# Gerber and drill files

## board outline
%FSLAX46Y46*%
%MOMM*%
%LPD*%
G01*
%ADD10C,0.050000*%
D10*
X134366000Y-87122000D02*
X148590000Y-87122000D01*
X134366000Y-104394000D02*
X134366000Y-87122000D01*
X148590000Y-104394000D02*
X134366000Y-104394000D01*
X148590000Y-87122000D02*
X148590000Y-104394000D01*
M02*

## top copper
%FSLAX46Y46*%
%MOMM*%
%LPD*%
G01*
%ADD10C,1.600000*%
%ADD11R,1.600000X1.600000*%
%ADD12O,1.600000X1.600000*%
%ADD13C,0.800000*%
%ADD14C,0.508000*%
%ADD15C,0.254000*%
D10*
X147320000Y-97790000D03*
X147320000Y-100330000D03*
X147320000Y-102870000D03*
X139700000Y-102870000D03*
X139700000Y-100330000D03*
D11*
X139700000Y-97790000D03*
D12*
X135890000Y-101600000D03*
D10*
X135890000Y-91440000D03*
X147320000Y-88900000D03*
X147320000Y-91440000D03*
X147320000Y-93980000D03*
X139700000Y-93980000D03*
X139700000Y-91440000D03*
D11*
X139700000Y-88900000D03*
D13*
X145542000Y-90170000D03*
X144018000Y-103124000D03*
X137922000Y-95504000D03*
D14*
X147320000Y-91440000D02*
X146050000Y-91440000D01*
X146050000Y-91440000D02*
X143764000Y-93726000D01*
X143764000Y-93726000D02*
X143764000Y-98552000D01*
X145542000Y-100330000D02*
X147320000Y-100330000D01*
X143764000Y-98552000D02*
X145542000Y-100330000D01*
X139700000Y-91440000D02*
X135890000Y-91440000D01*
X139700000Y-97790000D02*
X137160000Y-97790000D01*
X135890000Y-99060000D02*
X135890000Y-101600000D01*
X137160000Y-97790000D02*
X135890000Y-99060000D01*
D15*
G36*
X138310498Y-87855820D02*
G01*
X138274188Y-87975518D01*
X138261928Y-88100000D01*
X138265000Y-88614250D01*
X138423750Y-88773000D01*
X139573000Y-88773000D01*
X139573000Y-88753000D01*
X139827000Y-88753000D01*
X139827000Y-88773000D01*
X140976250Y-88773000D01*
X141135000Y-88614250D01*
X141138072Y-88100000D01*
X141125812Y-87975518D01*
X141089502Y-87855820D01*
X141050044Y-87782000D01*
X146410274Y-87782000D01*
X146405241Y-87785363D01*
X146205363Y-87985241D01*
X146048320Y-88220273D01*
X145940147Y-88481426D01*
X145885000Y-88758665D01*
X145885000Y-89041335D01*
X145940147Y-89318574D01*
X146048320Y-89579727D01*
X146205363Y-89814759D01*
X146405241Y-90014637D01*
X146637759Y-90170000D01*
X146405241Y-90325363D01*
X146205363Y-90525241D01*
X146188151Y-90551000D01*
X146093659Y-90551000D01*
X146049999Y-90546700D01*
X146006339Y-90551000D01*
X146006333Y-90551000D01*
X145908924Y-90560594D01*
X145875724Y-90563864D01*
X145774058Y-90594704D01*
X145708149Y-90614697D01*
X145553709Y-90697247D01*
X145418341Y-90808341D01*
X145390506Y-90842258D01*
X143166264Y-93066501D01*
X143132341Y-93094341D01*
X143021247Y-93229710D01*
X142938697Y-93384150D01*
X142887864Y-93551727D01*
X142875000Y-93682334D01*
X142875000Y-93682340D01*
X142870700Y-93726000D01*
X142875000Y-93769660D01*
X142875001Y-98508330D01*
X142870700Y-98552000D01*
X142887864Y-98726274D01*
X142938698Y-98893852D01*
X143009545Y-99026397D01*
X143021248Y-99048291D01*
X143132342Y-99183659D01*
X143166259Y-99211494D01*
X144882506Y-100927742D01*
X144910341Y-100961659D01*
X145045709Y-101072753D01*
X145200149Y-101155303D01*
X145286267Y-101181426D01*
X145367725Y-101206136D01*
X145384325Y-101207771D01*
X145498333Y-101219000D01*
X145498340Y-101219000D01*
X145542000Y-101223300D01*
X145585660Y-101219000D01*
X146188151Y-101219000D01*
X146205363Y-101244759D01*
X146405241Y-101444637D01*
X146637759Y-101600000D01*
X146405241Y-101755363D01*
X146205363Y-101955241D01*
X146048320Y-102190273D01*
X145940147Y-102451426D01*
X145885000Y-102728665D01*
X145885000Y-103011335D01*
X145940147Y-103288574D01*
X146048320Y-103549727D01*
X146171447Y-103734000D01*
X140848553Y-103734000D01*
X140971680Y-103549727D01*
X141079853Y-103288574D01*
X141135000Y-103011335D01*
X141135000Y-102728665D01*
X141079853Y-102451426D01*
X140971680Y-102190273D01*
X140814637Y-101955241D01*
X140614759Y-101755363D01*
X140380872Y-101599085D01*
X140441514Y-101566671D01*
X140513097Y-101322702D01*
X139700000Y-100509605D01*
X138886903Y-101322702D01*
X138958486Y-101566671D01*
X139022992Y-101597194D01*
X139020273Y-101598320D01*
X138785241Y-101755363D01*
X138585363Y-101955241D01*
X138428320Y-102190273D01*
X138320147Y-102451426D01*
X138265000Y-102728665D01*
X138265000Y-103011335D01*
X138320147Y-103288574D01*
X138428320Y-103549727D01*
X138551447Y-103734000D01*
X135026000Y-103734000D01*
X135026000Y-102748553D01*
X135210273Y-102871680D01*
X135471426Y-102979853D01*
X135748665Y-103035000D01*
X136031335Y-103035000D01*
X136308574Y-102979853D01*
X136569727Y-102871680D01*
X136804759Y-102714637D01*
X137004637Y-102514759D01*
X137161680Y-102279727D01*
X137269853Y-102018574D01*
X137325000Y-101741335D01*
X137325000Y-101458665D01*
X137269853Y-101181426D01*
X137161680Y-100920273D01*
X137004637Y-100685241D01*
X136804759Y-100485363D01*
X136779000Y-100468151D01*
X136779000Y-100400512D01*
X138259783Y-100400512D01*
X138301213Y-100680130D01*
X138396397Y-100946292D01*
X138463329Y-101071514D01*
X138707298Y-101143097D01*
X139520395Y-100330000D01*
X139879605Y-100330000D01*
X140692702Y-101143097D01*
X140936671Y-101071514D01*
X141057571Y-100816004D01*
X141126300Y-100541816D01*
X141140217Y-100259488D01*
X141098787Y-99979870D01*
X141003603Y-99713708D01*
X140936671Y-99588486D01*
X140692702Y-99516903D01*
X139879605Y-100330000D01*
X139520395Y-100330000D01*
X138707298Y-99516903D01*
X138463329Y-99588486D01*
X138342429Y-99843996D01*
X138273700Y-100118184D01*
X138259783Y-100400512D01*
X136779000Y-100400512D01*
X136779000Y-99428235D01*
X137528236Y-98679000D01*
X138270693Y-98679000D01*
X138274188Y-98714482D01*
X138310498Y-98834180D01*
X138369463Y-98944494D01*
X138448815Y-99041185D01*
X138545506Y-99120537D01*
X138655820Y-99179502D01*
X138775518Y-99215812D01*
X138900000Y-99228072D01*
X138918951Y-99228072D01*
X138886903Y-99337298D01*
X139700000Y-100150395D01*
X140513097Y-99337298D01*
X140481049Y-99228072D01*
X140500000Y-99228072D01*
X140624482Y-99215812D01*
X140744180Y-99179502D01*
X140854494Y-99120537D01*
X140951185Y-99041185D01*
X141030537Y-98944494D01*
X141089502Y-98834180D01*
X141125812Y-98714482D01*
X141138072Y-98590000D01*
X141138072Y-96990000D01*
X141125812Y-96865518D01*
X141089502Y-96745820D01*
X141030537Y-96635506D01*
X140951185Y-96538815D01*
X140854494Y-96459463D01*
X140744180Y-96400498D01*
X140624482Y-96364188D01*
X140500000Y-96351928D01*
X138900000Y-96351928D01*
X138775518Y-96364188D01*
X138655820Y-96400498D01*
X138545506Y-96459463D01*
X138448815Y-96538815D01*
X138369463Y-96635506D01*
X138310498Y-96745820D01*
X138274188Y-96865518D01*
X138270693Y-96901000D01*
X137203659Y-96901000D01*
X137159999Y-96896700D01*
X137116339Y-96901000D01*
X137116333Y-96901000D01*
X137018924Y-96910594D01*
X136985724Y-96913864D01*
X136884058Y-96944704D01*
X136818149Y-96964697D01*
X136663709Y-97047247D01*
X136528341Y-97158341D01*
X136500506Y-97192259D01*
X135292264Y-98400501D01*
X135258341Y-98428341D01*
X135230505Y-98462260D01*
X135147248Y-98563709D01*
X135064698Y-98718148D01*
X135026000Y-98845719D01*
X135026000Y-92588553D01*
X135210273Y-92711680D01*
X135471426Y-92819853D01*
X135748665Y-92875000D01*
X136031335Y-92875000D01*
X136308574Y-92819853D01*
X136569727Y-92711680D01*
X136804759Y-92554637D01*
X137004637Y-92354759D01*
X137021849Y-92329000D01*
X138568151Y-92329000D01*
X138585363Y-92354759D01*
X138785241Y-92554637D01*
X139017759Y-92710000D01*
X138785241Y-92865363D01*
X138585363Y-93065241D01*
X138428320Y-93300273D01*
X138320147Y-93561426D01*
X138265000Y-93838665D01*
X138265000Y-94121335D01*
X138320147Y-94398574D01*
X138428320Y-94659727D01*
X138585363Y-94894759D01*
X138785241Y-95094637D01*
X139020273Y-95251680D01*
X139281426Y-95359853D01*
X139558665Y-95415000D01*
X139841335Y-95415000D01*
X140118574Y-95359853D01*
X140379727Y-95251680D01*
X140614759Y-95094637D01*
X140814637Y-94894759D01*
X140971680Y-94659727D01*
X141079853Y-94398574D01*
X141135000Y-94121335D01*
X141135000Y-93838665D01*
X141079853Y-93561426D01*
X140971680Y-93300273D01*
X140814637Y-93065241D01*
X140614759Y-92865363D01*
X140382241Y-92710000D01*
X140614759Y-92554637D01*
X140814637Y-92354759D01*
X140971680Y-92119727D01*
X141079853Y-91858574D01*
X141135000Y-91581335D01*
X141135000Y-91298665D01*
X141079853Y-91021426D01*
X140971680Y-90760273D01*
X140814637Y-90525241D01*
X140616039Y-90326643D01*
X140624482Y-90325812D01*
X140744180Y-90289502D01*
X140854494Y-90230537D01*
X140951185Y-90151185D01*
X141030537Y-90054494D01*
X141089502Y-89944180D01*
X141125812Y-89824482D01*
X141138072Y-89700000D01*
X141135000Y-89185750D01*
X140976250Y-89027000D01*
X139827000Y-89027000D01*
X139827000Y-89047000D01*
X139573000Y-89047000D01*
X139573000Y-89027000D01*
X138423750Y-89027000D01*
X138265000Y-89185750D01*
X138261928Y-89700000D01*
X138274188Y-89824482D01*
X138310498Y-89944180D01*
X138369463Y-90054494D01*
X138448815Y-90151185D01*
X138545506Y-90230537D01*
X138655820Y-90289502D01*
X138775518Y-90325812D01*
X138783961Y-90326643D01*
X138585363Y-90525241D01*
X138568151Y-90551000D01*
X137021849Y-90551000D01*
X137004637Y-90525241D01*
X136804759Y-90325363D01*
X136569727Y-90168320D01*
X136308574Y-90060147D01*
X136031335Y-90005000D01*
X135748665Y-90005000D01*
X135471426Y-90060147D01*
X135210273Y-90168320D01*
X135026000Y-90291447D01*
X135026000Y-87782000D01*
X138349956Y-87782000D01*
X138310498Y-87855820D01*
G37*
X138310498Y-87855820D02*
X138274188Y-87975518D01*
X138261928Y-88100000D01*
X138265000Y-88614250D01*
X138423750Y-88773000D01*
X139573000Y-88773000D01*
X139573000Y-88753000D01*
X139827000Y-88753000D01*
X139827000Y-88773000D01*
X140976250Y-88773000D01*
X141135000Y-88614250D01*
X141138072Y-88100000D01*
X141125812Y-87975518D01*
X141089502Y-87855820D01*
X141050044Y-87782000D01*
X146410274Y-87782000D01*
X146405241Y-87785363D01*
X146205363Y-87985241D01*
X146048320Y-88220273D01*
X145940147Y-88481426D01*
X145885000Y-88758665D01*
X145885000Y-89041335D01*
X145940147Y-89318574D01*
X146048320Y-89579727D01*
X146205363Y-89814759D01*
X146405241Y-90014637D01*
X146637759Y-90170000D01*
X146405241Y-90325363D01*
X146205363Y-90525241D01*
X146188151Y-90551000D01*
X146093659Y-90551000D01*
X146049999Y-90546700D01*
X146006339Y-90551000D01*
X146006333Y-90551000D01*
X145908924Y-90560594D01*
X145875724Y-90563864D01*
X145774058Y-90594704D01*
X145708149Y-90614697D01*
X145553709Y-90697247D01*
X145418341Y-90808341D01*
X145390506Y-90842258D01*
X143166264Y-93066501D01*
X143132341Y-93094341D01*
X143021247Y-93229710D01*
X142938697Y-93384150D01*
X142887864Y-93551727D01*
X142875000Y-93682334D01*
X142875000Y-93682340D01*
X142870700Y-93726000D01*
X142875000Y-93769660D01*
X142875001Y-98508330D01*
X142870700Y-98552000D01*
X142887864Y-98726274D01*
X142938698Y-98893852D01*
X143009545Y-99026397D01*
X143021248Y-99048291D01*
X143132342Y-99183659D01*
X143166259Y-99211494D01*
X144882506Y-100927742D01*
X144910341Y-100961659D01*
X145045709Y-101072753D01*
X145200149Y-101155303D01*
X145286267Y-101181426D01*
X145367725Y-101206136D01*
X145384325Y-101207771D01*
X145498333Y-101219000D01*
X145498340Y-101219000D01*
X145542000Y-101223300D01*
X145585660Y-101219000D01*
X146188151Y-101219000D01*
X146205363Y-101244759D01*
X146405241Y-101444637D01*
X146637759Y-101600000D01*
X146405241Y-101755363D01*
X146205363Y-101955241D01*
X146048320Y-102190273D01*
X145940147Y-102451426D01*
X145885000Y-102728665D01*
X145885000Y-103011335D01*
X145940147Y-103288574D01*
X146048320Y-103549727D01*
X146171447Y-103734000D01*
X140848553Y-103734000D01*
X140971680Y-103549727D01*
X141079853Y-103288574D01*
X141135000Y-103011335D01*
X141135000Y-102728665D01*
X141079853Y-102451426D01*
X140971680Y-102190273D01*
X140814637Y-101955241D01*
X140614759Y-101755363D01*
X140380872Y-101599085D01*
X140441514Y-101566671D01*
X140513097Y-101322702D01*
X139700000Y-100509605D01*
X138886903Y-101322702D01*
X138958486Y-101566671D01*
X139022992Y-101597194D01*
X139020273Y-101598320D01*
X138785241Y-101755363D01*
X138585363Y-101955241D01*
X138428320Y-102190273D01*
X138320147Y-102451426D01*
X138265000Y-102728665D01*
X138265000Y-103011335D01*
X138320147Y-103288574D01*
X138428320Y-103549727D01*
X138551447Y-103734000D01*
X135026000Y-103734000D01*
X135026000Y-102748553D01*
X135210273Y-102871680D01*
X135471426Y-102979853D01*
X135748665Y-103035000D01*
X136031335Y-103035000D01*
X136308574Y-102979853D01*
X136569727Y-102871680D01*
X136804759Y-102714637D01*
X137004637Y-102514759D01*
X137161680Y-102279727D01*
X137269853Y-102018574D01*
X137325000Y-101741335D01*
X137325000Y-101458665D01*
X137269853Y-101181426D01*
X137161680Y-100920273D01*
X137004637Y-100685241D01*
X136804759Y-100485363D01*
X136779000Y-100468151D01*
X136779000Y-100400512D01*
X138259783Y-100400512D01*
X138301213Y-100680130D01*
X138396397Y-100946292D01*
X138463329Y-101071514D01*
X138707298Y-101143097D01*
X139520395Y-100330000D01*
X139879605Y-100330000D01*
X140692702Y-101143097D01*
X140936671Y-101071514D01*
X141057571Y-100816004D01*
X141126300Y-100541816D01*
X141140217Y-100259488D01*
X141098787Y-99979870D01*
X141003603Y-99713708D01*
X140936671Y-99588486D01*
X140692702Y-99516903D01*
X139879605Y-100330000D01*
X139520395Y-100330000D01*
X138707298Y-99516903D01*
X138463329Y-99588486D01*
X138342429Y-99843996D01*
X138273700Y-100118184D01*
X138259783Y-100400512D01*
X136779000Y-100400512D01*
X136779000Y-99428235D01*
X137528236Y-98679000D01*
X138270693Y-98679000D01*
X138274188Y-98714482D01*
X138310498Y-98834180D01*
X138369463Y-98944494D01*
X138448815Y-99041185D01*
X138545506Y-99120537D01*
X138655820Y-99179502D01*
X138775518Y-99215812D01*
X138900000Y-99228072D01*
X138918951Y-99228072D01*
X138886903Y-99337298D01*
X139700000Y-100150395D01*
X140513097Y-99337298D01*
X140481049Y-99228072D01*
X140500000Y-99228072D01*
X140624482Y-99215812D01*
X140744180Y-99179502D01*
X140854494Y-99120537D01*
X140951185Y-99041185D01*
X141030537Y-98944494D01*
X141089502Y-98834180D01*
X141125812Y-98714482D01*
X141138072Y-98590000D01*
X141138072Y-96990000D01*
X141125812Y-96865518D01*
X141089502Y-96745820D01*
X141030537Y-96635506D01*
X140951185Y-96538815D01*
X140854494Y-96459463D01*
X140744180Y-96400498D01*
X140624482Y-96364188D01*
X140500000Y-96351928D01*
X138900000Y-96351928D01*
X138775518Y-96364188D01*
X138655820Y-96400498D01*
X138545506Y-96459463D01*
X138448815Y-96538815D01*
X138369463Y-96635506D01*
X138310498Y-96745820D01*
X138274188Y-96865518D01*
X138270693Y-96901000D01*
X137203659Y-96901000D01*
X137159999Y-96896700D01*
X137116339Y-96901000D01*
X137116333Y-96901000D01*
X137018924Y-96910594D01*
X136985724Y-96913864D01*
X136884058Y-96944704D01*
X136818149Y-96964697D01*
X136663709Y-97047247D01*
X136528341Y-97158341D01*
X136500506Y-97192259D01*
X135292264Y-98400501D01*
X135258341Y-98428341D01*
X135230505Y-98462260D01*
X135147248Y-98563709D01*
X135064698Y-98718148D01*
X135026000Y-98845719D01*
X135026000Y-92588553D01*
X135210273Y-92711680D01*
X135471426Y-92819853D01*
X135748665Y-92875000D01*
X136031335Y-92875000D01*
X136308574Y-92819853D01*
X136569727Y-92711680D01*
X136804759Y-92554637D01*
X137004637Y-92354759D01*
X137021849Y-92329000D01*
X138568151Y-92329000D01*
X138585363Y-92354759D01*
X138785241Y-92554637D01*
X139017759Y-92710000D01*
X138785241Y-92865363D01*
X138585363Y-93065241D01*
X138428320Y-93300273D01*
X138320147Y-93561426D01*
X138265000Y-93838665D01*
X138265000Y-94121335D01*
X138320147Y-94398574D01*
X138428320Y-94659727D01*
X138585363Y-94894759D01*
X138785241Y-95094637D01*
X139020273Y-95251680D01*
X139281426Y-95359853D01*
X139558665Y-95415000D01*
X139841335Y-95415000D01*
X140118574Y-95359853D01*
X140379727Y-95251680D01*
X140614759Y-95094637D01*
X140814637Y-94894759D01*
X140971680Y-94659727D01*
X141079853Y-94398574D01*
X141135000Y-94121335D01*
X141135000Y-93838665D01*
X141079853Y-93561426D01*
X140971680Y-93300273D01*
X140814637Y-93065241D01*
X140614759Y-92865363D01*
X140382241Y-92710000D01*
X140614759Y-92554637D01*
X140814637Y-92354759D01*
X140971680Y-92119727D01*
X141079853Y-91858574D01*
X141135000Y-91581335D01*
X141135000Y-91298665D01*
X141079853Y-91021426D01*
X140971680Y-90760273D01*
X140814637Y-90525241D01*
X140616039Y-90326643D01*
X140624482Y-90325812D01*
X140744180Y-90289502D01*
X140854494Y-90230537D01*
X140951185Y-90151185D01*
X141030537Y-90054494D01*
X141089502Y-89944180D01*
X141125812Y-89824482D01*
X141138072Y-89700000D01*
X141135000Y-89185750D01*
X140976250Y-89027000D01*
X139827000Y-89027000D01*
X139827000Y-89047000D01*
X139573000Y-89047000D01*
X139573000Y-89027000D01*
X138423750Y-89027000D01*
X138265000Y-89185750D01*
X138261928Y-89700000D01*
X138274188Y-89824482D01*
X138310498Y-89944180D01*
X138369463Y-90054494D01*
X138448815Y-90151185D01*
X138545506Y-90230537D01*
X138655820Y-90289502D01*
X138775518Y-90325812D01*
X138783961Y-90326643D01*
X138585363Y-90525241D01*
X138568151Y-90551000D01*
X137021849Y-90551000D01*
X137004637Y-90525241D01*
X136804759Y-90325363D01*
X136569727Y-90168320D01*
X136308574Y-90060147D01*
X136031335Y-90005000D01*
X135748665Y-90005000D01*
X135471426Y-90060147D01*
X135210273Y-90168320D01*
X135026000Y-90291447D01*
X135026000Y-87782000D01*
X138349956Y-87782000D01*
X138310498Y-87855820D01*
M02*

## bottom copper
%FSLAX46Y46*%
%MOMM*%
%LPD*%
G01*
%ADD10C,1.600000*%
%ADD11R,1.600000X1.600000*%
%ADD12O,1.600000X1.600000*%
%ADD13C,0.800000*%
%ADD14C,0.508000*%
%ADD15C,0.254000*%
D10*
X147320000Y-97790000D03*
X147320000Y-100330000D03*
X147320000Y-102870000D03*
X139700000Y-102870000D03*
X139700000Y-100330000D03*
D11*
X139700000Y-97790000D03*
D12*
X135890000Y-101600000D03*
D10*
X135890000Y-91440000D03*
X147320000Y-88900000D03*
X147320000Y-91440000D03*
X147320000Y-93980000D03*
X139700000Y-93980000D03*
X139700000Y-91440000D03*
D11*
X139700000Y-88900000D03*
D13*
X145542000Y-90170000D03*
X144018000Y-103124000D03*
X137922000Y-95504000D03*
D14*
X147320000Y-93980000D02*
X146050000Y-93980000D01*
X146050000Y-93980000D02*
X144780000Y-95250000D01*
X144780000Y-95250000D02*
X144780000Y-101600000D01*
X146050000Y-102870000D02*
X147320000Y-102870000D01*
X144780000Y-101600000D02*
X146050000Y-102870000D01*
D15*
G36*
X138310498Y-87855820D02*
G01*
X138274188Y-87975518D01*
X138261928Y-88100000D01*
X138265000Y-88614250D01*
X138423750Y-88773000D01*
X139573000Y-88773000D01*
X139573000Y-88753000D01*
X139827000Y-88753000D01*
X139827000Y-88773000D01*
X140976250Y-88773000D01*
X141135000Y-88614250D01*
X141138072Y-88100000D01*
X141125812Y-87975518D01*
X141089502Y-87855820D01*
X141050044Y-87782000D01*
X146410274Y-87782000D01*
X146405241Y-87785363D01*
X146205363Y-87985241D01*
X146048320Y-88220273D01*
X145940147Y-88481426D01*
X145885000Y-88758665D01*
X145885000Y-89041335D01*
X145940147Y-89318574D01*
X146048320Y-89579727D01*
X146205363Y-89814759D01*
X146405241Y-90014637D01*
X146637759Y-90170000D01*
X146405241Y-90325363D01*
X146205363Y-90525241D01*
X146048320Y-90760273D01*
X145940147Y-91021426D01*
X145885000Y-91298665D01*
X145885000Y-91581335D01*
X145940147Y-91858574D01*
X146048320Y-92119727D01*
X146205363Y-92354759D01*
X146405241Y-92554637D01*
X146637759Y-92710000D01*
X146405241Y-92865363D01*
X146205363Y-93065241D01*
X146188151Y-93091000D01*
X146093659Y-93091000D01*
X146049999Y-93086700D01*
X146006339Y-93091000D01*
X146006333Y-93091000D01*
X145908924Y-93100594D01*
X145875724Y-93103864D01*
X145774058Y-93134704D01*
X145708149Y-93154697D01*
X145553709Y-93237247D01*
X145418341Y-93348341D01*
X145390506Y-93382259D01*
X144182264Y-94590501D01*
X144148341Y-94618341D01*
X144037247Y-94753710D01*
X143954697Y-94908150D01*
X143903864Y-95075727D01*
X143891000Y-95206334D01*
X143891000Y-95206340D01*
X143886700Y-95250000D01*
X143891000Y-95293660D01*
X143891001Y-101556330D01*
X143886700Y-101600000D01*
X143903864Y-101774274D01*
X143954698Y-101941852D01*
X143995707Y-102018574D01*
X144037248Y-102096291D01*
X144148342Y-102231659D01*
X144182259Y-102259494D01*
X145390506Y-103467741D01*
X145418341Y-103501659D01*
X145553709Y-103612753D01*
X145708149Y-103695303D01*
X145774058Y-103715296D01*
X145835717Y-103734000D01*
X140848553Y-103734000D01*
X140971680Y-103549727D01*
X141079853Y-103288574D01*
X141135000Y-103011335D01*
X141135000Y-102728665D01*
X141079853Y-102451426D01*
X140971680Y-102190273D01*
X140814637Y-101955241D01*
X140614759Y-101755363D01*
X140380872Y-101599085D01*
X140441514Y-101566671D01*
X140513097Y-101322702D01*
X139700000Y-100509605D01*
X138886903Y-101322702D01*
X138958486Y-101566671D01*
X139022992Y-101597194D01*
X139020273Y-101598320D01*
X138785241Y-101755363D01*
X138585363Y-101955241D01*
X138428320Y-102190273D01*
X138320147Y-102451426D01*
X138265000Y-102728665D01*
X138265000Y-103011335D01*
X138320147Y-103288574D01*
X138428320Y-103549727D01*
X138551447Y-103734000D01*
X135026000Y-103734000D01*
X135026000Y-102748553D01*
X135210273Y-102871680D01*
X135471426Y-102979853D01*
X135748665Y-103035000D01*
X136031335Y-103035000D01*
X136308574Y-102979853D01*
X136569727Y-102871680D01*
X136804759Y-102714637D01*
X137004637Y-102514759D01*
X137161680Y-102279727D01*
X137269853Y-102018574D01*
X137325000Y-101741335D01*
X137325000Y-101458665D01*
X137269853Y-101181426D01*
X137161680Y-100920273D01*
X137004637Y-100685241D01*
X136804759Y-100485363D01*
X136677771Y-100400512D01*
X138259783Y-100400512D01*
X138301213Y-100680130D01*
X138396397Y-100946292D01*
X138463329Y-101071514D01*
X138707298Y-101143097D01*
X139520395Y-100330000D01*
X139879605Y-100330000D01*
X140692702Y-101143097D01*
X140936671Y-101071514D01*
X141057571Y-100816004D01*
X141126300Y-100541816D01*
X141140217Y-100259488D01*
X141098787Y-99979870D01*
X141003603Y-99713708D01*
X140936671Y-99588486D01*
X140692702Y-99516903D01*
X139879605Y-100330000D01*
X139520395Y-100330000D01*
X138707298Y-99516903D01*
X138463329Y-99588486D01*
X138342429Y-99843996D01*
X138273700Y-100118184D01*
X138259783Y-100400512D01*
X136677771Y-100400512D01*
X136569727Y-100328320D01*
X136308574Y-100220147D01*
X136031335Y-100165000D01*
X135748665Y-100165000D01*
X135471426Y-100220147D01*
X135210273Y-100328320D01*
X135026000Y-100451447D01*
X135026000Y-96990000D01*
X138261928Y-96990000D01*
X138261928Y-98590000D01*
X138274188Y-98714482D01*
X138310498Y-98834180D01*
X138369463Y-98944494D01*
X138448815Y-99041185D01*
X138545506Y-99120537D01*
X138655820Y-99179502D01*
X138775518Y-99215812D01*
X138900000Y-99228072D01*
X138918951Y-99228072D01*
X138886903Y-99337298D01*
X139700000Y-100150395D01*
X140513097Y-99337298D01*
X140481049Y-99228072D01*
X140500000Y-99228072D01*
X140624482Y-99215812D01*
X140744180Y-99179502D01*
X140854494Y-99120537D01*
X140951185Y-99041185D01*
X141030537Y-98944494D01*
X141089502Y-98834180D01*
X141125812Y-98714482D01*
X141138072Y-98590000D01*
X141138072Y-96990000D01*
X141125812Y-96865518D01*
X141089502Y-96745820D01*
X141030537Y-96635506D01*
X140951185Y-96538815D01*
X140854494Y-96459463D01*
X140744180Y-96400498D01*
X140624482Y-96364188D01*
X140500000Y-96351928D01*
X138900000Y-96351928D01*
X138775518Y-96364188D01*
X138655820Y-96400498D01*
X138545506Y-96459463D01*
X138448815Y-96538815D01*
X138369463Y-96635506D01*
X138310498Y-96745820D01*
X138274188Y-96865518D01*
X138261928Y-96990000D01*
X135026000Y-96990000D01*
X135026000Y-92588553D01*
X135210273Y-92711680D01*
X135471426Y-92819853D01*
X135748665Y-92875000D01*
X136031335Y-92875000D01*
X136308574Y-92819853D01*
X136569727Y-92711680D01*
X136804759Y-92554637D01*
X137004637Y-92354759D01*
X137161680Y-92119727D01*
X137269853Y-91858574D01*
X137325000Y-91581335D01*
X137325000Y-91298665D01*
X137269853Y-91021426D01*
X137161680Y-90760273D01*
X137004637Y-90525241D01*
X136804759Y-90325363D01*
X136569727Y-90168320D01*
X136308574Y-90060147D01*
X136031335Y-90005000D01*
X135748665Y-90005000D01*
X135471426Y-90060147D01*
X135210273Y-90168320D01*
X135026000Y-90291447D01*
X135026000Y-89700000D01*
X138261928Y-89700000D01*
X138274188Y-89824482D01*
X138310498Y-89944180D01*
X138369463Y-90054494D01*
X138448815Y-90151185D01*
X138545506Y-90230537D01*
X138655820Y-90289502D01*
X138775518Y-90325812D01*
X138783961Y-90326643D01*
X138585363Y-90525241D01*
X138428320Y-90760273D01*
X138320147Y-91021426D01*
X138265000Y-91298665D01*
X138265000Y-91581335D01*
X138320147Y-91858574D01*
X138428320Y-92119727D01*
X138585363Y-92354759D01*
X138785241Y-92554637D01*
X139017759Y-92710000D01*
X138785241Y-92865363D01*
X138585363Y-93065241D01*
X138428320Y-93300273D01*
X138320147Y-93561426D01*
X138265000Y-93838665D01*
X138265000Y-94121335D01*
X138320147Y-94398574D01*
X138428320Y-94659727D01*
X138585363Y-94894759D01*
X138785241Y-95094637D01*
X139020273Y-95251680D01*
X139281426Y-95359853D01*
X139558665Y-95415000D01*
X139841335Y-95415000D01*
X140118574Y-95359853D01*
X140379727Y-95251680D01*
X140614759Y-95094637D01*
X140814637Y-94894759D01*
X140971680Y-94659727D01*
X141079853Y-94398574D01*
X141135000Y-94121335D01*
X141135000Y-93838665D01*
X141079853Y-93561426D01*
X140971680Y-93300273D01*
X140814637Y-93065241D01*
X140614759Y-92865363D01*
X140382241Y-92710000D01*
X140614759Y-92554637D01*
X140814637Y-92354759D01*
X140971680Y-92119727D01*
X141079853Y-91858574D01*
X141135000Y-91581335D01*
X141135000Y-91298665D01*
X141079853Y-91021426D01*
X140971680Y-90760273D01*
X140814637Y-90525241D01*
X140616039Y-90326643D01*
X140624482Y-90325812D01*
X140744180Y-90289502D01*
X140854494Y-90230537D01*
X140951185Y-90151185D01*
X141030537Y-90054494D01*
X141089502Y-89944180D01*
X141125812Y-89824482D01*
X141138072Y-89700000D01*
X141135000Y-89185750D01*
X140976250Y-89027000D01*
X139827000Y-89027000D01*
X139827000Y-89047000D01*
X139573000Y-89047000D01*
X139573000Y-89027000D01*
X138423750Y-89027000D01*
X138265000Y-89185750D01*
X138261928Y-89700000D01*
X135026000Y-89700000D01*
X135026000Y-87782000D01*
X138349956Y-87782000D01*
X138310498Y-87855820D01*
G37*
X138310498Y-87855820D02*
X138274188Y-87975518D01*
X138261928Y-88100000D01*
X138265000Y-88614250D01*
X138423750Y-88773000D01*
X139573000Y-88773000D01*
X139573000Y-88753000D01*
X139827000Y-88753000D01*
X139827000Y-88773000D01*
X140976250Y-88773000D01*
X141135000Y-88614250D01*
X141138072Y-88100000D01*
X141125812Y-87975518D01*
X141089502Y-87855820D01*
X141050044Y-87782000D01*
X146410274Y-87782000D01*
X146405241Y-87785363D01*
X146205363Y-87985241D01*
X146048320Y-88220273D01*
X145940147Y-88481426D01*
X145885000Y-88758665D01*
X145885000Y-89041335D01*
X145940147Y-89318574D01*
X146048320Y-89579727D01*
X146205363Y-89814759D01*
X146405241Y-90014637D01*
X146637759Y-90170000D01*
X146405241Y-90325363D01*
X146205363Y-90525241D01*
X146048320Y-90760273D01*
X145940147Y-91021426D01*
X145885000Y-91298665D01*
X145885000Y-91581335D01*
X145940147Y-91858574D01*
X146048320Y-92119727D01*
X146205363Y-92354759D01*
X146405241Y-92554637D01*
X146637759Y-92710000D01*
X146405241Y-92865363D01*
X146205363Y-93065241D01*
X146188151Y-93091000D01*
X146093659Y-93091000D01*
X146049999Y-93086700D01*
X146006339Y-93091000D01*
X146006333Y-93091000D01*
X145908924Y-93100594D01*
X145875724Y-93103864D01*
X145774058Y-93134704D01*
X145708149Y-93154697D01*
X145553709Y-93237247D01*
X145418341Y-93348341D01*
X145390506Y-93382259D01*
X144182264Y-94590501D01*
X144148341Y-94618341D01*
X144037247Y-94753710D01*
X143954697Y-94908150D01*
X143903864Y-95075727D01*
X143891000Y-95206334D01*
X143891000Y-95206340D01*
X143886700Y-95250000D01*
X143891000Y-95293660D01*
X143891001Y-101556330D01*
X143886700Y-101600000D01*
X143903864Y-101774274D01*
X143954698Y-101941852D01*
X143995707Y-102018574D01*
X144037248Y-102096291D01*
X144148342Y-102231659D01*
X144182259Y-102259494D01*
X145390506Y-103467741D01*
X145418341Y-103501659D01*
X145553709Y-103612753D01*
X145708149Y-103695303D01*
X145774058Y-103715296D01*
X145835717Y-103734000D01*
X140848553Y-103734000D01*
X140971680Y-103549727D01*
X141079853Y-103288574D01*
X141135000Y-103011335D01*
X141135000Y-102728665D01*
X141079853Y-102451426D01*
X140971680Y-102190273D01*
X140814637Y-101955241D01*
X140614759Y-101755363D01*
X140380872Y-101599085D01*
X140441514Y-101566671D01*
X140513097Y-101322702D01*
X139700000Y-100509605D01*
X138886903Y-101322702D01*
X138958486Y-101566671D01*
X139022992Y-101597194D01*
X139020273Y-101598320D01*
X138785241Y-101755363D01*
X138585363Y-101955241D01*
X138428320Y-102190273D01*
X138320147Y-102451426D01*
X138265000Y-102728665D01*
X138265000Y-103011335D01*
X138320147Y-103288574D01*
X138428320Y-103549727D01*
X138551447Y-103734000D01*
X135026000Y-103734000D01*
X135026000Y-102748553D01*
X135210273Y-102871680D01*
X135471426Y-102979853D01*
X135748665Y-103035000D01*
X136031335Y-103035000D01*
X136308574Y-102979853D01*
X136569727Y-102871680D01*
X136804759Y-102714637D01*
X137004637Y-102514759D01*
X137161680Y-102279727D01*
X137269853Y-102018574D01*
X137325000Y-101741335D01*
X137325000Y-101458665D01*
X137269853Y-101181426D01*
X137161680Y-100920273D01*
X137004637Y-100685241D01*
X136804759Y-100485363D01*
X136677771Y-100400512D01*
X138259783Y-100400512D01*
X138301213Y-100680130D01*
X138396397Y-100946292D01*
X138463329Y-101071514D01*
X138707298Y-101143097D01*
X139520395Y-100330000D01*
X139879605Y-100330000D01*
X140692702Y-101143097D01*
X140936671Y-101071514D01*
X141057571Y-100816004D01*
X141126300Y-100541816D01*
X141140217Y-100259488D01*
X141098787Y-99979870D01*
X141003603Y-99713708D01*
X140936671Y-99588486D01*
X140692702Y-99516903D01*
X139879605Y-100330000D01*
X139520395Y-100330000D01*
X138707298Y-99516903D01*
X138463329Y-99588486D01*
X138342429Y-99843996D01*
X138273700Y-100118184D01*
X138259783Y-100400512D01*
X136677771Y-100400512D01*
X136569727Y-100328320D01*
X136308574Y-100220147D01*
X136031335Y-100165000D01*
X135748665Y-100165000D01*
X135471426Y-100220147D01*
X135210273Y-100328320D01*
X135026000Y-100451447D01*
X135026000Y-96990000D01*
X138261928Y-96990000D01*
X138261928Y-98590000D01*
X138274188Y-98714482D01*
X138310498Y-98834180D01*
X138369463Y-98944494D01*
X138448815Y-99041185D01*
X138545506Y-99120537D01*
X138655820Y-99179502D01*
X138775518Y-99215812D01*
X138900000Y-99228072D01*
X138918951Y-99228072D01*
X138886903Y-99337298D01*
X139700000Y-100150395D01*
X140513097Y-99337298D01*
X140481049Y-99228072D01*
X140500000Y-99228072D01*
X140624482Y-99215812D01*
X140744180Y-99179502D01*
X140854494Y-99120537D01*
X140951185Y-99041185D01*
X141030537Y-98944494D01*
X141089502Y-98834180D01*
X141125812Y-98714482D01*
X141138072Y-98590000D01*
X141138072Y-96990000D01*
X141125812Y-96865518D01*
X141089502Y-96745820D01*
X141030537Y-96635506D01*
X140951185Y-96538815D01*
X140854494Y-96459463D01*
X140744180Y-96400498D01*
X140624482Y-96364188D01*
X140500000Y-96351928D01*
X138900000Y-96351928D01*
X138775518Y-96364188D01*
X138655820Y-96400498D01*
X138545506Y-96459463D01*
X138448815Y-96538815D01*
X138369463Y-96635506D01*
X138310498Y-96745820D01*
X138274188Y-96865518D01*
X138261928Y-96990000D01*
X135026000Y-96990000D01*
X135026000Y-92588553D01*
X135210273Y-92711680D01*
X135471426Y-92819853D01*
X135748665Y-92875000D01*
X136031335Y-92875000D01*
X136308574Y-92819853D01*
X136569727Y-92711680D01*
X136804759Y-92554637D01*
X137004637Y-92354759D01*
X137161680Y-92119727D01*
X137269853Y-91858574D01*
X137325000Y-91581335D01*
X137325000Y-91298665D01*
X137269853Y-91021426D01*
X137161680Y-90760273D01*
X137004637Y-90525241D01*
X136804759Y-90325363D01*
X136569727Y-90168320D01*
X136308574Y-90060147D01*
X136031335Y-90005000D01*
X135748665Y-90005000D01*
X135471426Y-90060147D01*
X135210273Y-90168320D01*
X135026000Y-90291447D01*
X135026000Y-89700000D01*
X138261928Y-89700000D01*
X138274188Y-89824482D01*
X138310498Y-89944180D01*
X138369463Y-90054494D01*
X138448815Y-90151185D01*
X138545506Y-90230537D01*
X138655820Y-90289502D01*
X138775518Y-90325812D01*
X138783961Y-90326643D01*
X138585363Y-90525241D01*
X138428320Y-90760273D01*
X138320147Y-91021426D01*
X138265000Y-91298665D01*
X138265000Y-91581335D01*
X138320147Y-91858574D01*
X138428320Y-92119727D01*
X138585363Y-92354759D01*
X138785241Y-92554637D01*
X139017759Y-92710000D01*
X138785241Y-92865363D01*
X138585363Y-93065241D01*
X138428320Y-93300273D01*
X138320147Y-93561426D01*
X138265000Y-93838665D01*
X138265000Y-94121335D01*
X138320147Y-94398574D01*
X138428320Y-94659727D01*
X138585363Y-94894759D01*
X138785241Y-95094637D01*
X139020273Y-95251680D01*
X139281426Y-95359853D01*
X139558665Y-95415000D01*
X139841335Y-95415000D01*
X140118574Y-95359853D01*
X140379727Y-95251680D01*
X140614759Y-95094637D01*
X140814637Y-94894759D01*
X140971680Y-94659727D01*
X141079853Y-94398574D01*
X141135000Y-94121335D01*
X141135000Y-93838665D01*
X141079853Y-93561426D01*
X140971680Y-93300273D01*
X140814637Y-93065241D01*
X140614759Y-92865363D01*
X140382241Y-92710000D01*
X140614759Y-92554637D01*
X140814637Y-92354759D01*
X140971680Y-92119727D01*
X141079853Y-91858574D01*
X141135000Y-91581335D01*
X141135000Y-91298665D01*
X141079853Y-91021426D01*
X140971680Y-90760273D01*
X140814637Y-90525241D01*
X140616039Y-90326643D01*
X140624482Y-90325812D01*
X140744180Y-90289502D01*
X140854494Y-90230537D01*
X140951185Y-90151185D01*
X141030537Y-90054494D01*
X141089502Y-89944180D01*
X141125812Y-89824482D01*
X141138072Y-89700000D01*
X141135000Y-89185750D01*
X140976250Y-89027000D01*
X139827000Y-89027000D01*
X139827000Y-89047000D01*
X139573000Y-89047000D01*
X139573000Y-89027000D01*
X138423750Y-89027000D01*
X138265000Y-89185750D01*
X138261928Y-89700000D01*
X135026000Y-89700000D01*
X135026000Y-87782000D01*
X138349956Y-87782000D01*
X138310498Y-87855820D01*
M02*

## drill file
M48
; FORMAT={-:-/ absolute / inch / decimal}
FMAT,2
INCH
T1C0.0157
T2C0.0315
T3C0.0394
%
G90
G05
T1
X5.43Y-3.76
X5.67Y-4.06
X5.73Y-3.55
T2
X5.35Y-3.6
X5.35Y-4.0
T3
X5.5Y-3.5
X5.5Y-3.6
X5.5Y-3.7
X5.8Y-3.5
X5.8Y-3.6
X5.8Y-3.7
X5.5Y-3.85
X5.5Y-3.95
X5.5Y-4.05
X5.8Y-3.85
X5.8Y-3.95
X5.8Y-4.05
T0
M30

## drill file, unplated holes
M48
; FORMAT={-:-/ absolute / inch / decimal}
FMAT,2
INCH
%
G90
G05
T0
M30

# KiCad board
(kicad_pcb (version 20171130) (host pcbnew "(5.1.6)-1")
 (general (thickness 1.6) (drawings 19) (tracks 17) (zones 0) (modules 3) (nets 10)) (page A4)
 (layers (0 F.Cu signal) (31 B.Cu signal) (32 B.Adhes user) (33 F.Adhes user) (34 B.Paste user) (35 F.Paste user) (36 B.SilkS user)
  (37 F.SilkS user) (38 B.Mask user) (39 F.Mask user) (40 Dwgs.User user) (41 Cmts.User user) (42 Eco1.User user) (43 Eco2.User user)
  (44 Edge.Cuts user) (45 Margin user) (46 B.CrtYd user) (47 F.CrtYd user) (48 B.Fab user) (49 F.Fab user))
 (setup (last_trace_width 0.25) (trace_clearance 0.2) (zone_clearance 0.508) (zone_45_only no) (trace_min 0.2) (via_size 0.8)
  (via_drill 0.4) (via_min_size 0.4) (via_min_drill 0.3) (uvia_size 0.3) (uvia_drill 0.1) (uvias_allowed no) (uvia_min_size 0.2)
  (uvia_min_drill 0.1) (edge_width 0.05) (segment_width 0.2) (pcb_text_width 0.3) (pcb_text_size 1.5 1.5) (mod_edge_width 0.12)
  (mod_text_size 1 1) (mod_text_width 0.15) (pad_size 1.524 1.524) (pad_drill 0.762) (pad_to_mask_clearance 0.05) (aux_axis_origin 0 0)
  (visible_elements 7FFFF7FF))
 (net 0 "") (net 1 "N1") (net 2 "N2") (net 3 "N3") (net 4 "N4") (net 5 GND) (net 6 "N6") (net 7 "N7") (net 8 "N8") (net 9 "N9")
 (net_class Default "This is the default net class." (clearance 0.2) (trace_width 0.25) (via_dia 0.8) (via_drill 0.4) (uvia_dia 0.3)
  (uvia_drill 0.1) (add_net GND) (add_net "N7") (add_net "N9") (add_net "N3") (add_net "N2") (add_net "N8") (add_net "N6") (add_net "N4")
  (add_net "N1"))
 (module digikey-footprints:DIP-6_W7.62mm (layer F.Cu) (at 139.7 97.79)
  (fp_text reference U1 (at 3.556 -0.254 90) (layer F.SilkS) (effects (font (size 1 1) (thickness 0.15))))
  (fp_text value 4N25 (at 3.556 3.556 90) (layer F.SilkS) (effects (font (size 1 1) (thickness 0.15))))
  (pad 6 thru_hole circle (at 7.62 0) (size 1.6 1.6) (drill 1) (layers *.Cu *.Mask) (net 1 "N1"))
  (pad 5 thru_hole circle (at 7.62 2.54) (size 1.6 1.6) (drill 1) (layers *.Cu *.Mask) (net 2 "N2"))
  (pad 4 thru_hole circle (at 7.62 5.08) (size 1.6 1.6) (drill 1) (layers *.Cu *.Mask) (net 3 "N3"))
  (pad 3 thru_hole circle (at 0 5.08) (size 1.6 1.6) (drill 1) (layers *.Cu *.Mask) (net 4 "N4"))
  (pad 2 thru_hole circle (at 0 2.54) (size 1.6 1.6) (drill 1) (layers *.Cu *.Mask) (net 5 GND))
  (pad 1 thru_hole rect (at 0 0) (size 1.6 1.6) (drill 1) (layers *.Cu *.Mask) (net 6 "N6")))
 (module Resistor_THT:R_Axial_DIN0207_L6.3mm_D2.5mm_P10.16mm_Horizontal (layer F.Cu) (at 135.89 91.44 270)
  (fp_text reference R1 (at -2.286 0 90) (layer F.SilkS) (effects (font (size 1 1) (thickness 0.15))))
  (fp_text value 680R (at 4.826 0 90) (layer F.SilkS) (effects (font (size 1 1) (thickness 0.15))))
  (pad 2 thru_hole oval (at 10.16 0 270) (size 1.6 1.6) (drill 0.8) (layers *.Cu *.Mask) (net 6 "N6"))
  (pad 1 thru_hole circle (at 0 0 270) (size 1.6 1.6) (drill 0.8) (layers *.Cu *.Mask) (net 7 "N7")))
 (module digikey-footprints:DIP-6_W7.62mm (layer F.Cu) (at 139.7 88.9)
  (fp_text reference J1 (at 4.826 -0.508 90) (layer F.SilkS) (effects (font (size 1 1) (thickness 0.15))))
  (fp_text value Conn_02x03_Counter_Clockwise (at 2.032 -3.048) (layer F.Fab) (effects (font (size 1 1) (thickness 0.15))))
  (pad 6 thru_hole circle (at 7.62 0) (size 1.6 1.6) (drill 1) (layers *.Cu *.Mask) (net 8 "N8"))
  (pad 5 thru_hole circle (at 7.62 2.54) (size 1.6 1.6) (drill 1) (layers *.Cu *.Mask) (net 2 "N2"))
  (pad 4 thru_hole circle (at 7.62 5.08) (size 1.6 1.6) (drill 1) (layers *.Cu *.Mask) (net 3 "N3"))
  (pad 3 thru_hole circle (at 0 5.08) (size 1.6 1.6) (drill 1) (layers *.Cu *.Mask) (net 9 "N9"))
  (pad 2 thru_hole circle (at 0 2.54) (size 1.6 1.6) (drill 1) (layers *.Cu *.Mask) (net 7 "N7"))
  (pad 1 thru_hole rect (at 0 0) (size 1.6 1.6) (drill 1) (layers *.Cu *.Mask) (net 5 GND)))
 (gr_line (start 134.366 87.122) (end 148.59 87.122) (layer Edge.Cuts) (width 0.05))
 (gr_line (start 134.366 104.394) (end 134.366 87.122) (layer Edge.Cuts) (width 0.05))
 (gr_line (start 148.59 104.394) (end 134.366 104.394) (layer Edge.Cuts) (width 0.05))
 (gr_line (start 148.59 87.122) (end 148.59 104.394) (layer Edge.Cuts) (width 0.05))
 (segment (start 147.32 91.44) (end 146.05 91.44) (width 0.508) (layer F.Cu) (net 2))
 (segment (start 146.05 91.44) (end 143.764 93.726) (width 0.508) (layer F.Cu) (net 2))
 (segment (start 143.764 93.726) (end 143.764 98.552) (width 0.508) (layer F.Cu) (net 2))
 (segment (start 145.542 100.33) (end 147.32 100.33) (width 0.508) (layer F.Cu) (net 2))
 (segment (start 143.764 98.552) (end 145.542 100.33) (width 0.508) (layer F.Cu) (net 2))
 (segment (start 147.32 93.98) (end 146.05 93.98) (width 0.508) (layer B.Cu) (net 3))
 (segment (start 146.05 93.98) (end 144.78 95.25) (width 0.508) (layer B.Cu) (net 3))
 (segment (start 144.78 95.25) (end 144.78 101.6) (width 0.508) (layer B.Cu) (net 3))
 (segment (start 146.05 102.87) (end 147.32 102.87) (width 0.508) (layer B.Cu) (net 3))
 (segment (start 144.78 101.6) (end 146.05 102.87) (width 0.508) (layer B.Cu) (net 3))
 (segment (start 139.7 91.44) (end 135.89 91.44) (width 0.508) (layer F.Cu) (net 7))
 (via (at 145.542 90.17) (size 0.8) (drill 0.4) (layers F.Cu B.Cu) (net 5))
 (via (at 144.018 103.124) (size 0.8) (drill 0.4) (layers F.Cu B.Cu) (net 5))
 (via (at 137.922 95.504) (size 0.8) (drill 0.4) (layers F.Cu B.Cu) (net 5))
 (segment (start 139.7 97.79) (end 137.16 97.79) (width 0.508) (layer F.Cu) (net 6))
 (segment (start 135.89 99.06) (end 135.89 101.6) (width 0.508) (layer F.Cu) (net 6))
 (segment (start 137.16 97.79) (end 135.89 99.06) (width 0.508) (layer F.Cu) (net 6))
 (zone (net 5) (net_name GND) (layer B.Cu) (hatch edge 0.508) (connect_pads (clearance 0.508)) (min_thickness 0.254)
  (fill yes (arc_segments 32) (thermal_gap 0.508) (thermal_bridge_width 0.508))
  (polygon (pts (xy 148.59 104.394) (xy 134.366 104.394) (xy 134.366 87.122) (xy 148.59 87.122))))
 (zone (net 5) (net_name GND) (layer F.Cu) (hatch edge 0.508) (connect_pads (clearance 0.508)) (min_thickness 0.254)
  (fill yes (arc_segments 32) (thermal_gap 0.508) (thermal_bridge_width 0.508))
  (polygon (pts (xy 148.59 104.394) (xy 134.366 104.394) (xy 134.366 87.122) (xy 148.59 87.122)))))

